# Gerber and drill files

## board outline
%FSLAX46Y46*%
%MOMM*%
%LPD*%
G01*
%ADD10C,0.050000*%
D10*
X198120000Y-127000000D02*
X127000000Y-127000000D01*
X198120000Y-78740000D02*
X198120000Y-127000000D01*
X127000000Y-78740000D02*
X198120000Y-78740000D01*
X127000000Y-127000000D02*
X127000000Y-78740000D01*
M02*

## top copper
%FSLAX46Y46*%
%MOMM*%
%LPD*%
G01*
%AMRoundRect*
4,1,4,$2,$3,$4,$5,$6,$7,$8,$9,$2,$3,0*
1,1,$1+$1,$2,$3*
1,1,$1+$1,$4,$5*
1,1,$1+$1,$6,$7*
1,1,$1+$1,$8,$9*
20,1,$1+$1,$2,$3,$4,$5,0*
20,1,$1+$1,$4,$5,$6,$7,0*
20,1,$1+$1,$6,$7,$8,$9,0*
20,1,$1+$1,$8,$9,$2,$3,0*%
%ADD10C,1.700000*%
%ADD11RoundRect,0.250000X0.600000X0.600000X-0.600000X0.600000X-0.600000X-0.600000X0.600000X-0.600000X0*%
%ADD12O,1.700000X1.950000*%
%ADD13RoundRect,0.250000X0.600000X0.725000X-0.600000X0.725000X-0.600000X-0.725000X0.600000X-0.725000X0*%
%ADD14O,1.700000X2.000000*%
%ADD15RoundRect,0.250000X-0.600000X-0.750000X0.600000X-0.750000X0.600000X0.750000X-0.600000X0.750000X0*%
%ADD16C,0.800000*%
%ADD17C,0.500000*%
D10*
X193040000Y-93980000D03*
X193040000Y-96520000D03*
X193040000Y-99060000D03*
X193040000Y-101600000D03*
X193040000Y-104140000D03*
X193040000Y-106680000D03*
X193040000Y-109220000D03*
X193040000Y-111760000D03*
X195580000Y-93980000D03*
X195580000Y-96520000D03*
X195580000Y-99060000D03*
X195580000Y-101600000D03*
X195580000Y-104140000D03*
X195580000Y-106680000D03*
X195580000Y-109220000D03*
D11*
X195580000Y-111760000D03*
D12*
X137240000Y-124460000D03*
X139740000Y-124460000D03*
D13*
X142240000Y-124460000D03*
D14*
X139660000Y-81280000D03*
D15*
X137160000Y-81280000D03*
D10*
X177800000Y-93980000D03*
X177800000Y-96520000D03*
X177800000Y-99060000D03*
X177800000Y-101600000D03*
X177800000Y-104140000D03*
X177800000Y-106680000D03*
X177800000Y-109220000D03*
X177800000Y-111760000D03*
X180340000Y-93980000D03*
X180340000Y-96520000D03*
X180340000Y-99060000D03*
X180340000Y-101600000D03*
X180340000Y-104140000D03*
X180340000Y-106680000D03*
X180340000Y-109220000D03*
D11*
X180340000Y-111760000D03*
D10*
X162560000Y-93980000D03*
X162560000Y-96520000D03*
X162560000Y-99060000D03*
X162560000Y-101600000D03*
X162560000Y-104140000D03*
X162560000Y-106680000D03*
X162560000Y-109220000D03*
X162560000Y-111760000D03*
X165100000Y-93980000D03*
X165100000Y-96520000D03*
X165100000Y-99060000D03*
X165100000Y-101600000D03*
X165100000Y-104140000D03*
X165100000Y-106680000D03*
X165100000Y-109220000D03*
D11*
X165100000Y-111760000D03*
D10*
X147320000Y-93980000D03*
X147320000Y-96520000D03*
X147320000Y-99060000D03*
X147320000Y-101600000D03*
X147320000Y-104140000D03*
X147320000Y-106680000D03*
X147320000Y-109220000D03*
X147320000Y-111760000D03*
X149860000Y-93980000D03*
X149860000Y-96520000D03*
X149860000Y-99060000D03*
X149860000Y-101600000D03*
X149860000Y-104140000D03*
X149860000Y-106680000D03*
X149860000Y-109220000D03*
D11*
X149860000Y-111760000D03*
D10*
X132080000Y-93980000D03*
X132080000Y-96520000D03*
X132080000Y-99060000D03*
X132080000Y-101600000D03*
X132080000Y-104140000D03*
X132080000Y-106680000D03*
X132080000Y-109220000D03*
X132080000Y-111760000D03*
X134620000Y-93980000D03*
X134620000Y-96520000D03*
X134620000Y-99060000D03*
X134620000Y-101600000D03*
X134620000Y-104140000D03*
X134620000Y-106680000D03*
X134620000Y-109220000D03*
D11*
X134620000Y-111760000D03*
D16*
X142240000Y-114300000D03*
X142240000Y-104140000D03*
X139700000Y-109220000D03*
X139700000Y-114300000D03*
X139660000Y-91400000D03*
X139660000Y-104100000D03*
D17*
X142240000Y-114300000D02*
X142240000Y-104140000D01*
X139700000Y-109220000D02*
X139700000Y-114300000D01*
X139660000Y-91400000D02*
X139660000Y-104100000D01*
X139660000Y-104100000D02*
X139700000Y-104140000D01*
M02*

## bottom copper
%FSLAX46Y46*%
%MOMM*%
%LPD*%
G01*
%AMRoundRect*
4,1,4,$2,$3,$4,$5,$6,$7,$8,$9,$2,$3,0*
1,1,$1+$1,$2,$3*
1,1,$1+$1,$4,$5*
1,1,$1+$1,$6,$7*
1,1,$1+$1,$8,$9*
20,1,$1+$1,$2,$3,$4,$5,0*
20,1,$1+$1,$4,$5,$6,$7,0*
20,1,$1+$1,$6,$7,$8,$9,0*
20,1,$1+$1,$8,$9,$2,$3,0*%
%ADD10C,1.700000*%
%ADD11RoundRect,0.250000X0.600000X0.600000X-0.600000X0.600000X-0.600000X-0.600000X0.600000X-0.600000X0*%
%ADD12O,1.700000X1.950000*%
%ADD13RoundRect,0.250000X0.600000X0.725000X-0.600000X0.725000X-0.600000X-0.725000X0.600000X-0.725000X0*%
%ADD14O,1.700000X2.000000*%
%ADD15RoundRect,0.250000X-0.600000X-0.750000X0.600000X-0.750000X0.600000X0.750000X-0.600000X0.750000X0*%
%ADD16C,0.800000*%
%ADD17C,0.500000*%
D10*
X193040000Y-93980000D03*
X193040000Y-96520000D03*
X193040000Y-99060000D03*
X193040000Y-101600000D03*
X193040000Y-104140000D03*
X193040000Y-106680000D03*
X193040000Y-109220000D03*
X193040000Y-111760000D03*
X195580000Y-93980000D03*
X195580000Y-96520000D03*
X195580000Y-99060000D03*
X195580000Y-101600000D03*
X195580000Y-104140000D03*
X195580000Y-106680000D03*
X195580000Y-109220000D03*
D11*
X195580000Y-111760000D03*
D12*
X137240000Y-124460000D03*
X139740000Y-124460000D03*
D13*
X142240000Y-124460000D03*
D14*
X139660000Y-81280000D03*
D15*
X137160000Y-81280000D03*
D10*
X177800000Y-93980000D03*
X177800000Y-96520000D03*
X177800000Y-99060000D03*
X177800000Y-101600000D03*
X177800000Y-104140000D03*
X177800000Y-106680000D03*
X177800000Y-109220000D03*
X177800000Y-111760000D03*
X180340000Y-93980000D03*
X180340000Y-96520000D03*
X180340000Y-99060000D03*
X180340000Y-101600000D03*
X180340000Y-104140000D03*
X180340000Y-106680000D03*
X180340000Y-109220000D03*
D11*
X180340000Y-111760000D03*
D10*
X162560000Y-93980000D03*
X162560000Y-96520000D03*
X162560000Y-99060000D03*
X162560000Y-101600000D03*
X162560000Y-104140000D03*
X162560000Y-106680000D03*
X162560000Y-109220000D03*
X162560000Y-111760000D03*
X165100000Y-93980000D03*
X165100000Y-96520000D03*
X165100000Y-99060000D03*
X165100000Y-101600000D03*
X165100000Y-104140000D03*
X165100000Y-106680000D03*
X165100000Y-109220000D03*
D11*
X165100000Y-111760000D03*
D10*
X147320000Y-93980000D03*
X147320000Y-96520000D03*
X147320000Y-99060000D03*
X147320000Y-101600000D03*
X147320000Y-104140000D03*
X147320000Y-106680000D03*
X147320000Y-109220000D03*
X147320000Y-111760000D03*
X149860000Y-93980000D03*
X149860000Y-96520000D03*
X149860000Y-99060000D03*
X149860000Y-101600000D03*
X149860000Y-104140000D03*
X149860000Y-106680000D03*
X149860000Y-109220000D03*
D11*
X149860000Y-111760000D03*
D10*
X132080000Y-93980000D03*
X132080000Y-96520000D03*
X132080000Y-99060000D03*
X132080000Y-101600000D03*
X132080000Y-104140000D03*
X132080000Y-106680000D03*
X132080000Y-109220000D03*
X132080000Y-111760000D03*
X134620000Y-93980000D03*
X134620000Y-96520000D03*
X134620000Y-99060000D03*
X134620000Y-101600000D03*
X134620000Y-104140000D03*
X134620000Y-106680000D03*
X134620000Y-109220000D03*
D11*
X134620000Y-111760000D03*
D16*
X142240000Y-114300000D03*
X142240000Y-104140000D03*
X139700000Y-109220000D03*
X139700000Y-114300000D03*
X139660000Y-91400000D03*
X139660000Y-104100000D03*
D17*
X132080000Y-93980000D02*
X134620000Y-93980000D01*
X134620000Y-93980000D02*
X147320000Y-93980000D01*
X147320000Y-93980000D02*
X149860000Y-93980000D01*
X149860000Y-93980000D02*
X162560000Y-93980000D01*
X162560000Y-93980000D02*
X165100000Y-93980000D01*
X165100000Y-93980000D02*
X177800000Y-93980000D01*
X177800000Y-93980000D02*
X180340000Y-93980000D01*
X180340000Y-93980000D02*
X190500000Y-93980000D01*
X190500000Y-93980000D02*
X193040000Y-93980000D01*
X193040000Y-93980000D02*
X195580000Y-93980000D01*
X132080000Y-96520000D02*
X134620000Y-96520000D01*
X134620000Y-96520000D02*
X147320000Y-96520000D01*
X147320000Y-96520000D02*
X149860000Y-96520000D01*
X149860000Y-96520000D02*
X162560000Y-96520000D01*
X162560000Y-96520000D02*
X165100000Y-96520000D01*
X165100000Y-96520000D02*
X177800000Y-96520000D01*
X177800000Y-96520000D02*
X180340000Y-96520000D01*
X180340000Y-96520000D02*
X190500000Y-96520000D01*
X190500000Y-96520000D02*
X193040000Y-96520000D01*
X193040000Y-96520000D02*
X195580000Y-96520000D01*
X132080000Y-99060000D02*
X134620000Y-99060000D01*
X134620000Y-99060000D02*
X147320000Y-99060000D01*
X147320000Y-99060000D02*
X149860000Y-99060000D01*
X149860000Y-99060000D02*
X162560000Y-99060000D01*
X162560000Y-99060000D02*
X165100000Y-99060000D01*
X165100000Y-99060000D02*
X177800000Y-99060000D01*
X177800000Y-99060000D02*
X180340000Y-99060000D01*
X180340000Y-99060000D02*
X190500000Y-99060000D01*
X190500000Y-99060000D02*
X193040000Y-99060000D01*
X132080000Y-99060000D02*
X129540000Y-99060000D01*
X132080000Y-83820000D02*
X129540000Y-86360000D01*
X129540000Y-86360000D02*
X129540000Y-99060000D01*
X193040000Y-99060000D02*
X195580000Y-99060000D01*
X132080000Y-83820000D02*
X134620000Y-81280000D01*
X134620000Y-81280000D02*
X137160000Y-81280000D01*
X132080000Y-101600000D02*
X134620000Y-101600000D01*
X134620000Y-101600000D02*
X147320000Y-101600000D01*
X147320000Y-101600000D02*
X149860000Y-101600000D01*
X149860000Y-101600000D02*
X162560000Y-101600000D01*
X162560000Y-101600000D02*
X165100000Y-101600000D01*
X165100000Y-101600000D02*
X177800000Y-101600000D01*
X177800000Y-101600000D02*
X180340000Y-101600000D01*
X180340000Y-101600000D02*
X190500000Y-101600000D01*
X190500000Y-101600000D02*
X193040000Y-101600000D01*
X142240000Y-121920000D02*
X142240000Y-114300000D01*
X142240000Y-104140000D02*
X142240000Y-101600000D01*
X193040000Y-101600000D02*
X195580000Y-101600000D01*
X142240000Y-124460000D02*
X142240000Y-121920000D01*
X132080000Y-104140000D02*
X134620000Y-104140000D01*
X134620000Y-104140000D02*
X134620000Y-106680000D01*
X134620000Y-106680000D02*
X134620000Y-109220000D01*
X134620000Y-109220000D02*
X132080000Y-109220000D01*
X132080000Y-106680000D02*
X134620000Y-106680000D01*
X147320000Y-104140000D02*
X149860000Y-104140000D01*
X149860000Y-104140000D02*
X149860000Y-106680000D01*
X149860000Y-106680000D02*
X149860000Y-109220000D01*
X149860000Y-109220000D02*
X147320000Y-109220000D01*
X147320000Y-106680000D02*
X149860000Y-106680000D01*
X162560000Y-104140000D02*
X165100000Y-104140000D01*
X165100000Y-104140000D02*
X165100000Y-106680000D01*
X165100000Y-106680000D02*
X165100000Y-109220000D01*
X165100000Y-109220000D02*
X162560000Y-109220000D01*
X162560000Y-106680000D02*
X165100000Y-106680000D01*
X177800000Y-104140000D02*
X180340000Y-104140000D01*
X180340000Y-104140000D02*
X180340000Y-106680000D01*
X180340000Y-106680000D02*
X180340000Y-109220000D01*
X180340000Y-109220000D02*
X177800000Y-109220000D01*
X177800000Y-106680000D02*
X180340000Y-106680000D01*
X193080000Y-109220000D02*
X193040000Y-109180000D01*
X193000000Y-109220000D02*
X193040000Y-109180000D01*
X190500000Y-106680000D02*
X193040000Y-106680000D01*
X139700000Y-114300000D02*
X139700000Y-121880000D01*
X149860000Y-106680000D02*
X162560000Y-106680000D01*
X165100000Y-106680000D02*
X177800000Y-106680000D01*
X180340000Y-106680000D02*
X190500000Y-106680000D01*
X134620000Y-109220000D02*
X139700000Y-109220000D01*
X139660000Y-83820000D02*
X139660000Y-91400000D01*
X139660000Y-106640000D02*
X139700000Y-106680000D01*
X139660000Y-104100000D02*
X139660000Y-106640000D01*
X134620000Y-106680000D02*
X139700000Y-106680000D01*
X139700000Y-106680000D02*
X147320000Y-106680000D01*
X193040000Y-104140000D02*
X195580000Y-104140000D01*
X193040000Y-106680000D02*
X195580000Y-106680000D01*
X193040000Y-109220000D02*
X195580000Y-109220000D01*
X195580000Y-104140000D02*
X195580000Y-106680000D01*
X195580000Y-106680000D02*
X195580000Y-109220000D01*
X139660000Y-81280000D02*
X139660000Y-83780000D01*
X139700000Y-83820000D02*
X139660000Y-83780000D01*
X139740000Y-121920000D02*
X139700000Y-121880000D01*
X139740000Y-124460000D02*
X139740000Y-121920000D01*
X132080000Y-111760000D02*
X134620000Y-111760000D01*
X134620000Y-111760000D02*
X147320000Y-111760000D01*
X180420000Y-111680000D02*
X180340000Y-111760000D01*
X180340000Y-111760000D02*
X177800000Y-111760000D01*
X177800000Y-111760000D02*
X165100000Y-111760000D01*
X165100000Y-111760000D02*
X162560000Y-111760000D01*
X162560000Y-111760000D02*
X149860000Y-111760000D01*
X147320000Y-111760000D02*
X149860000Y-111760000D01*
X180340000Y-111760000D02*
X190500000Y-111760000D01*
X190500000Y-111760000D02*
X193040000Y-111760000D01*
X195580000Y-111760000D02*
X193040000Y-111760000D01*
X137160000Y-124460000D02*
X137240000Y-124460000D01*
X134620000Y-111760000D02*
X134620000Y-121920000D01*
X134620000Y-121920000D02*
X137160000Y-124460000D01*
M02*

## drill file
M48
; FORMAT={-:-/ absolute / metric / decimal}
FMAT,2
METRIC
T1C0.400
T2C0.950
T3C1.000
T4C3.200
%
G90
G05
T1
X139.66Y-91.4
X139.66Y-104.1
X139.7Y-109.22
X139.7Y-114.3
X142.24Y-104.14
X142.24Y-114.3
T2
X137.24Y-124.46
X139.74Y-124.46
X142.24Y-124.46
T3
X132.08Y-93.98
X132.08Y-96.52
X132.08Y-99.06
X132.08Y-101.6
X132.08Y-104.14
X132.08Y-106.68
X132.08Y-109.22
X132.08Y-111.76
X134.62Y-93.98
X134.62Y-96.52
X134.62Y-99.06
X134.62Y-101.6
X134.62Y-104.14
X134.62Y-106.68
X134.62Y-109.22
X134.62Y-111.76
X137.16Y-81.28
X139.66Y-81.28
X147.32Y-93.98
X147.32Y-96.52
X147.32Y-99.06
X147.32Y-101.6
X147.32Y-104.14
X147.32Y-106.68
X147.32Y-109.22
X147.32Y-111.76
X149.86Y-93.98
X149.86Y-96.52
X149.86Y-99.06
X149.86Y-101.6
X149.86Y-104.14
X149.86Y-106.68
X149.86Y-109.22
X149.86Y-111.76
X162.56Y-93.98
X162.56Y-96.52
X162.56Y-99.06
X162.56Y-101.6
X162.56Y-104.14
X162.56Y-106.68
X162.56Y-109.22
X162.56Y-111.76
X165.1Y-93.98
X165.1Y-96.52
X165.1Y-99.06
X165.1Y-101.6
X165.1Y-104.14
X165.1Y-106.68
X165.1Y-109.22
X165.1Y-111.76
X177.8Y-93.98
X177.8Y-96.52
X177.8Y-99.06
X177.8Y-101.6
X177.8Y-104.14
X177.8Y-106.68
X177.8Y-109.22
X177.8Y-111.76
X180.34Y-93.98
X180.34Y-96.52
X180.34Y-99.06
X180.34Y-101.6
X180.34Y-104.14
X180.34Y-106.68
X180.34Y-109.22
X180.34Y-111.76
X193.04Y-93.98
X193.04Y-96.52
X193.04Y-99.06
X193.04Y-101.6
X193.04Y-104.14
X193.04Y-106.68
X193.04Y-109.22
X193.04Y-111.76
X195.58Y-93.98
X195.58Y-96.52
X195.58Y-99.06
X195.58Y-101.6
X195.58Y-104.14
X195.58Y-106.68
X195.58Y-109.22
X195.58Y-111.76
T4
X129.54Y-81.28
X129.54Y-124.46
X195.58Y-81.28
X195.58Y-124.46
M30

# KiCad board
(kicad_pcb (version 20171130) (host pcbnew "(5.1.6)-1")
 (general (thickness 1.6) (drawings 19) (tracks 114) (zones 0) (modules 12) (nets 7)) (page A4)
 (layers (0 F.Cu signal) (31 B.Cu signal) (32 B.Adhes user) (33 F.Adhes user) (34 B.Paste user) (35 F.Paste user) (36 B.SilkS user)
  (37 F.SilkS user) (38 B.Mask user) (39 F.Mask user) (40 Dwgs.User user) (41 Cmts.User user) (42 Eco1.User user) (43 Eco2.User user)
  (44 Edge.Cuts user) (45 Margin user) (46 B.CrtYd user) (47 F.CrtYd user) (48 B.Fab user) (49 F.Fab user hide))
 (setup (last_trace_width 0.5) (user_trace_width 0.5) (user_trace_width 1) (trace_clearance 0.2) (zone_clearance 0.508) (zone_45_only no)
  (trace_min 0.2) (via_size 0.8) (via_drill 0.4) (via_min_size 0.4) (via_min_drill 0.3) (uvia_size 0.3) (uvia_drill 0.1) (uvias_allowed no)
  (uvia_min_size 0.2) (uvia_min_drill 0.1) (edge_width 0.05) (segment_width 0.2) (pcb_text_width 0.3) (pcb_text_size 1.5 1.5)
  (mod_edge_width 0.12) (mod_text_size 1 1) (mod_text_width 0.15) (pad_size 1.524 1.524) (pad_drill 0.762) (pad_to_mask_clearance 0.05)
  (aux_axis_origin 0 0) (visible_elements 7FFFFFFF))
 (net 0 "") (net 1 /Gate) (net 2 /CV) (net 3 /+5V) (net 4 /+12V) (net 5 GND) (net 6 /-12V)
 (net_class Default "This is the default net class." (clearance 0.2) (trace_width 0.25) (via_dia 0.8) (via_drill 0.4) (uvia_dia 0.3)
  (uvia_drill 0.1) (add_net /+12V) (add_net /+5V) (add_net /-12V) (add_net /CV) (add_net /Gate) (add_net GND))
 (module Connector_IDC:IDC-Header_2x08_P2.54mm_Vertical (layer F.Cu) (at 195.58 111.76 180)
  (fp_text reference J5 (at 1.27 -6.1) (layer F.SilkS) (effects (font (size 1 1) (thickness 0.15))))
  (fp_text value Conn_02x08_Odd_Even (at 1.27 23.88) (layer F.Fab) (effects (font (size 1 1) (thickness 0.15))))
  (pad 16 thru_hole circle (at 2.54 17.78 180) (size 1.7 1.7) (drill 1) (layers *.Cu *.Mask) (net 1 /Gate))
  (pad 14 thru_hole circle (at 2.54 15.24 180) (size 1.7 1.7) (drill 1) (layers *.Cu *.Mask) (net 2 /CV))
  (pad 12 thru_hole circle (at 2.54 12.7 180) (size 1.7 1.7) (drill 1) (layers *.Cu *.Mask) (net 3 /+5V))
  (pad 10 thru_hole circle (at 2.54 10.16 180) (size 1.7 1.7) (drill 1) (layers *.Cu *.Mask) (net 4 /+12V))
  (pad 8 thru_hole circle (at 2.54 7.62 180) (size 1.7 1.7) (drill 1) (layers *.Cu *.Mask) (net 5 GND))
  (pad 6 thru_hole circle (at 2.54 5.08 180) (size 1.7 1.7) (drill 1) (layers *.Cu *.Mask) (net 5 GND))
  (pad 4 thru_hole circle (at 2.54 2.54 180) (size 1.7 1.7) (drill 1) (layers *.Cu *.Mask) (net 5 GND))
  (pad 2 thru_hole circle (at 2.54 0 180) (size 1.7 1.7) (drill 1) (layers *.Cu *.Mask) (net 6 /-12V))
  (pad 15 thru_hole circle (at 0 17.78 180) (size 1.7 1.7) (drill 1) (layers *.Cu *.Mask) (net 1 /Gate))
  (pad 13 thru_hole circle (at 0 15.24 180) (size 1.7 1.7) (drill 1) (layers *.Cu *.Mask) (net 2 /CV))
  (pad 11 thru_hole circle (at 0 12.7 180) (size 1.7 1.7) (drill 1) (layers *.Cu *.Mask) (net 3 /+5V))
  (pad 9 thru_hole circle (at 0 10.16 180) (size 1.7 1.7) (drill 1) (layers *.Cu *.Mask) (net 4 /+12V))
  (pad 7 thru_hole circle (at 0 7.62 180) (size 1.7 1.7) (drill 1) (layers *.Cu *.Mask) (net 5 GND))
  (pad 5 thru_hole circle (at 0 5.08 180) (size 1.7 1.7) (drill 1) (layers *.Cu *.Mask) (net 5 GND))
  (pad 3 thru_hole circle (at 0 2.54 180) (size 1.7 1.7) (drill 1) (layers *.Cu *.Mask) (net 5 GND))
  (pad 1 thru_hole roundrect (at 0 0 180) (size 1.7 1.7) (drill 1) (layers *.Cu *.Mask) (roundrect_rratio 0.147059) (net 6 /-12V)))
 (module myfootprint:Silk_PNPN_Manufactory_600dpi (layer F.Cu) (at 182.88 83.82)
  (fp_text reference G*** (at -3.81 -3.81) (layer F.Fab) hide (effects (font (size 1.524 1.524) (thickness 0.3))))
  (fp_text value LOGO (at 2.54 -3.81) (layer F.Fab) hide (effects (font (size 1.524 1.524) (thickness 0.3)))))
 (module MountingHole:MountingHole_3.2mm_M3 (layer F.Cu) (at 195.58 124.46)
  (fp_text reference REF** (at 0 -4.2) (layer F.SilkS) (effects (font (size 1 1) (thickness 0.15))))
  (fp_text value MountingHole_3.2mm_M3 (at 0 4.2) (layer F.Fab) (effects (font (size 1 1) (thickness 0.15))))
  (pad 1 np_thru_hole circle (at 0 0) (size 3.2 3.2) (drill 3.2) (layers *.Cu *.Mask)))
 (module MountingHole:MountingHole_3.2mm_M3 (layer F.Cu) (at 129.54 124.46)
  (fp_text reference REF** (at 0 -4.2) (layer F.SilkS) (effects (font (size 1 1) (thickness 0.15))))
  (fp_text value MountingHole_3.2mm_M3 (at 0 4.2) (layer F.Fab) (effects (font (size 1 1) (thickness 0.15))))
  (pad 1 np_thru_hole circle (at 0 0) (size 3.2 3.2) (drill 3.2) (layers *.Cu *.Mask)))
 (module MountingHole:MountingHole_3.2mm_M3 (layer F.Cu) (at 195.58 81.28)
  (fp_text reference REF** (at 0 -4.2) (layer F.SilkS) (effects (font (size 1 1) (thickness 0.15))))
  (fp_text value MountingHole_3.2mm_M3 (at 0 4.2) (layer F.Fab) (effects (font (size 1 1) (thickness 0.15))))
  (pad 1 np_thru_hole circle (at 0 0) (size 3.2 3.2) (drill 3.2) (layers *.Cu *.Mask)))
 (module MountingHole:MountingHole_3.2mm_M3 (layer F.Cu) (at 129.54 81.28)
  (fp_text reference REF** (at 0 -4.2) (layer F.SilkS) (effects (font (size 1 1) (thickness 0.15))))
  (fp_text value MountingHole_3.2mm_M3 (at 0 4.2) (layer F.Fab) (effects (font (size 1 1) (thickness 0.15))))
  (pad 1 np_thru_hole circle (at 0 0) (size 3.2 3.2) (drill 3.2) (layers *.Cu *.Mask)))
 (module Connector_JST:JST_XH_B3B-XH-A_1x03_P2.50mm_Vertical (layer F.Cu) (at 142.24 124.46 180)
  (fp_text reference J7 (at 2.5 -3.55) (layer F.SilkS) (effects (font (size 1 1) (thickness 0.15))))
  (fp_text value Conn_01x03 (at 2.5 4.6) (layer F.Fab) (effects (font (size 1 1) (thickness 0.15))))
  (pad 3 thru_hole oval (at 5 0 180) (size 1.7 1.95) (drill 0.95) (layers *.Cu *.Mask) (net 6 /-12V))
  (pad 2 thru_hole oval (at 2.5 0 180) (size 1.7 1.95) (drill 0.95) (layers *.Cu *.Mask) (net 5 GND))
  (pad 1 thru_hole roundrect (at 0 0 180) (size 1.7 1.95) (drill 0.95) (layers *.Cu *.Mask) (roundrect_rratio 0.147059) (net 4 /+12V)))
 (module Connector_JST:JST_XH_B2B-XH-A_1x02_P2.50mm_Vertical (layer F.Cu) (at 137.16 81.28)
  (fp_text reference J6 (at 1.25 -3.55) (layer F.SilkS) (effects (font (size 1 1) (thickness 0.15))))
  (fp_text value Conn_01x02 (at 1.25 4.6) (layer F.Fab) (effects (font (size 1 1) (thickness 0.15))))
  (pad 2 thru_hole oval (at 2.5 0) (size 1.7 2) (drill 1) (layers *.Cu *.Mask) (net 5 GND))
  (pad 1 thru_hole roundrect (at 0 0) (size 1.7 2) (drill 1) (layers *.Cu *.Mask) (roundrect_rratio 0.147059) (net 3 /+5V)))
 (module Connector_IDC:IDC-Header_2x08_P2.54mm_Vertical (layer F.Cu) (at 180.34 111.76 180)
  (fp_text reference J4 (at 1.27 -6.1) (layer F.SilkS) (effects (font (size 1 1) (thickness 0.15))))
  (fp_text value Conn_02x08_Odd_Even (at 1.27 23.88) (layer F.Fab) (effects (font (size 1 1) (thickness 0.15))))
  (pad 16 thru_hole circle (at 2.54 17.78 180) (size 1.7 1.7) (drill 1) (layers *.Cu *.Mask) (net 1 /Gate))
  (pad 14 thru_hole circle (at 2.54 15.24 180) (size 1.7 1.7) (drill 1) (layers *.Cu *.Mask) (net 2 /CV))
  (pad 12 thru_hole circle (at 2.54 12.7 180) (size 1.7 1.7) (drill 1) (layers *.Cu *.Mask) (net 3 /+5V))
  (pad 10 thru_hole circle (at 2.54 10.16 180) (size 1.7 1.7) (drill 1) (layers *.Cu *.Mask) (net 4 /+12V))
  (pad 8 thru_hole circle (at 2.54 7.62 180) (size 1.7 1.7) (drill 1) (layers *.Cu *.Mask) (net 5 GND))
  (pad 6 thru_hole circle (at 2.54 5.08 180) (size 1.7 1.7) (drill 1) (layers *.Cu *.Mask) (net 5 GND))
  (pad 4 thru_hole circle (at 2.54 2.54 180) (size 1.7 1.7) (drill 1) (layers *.Cu *.Mask) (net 5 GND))
  (pad 2 thru_hole circle (at 2.54 0 180) (size 1.7 1.7) (drill 1) (layers *.Cu *.Mask) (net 6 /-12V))
  (pad 15 thru_hole circle (at 0 17.78 180) (size 1.7 1.7) (drill 1) (layers *.Cu *.Mask) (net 1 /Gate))
  (pad 13 thru_hole circle (at 0 15.24 180) (size 1.7 1.7) (drill 1) (layers *.Cu *.Mask) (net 2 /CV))
  (pad 11 thru_hole circle (at 0 12.7 180) (size 1.7 1.7) (drill 1) (layers *.Cu *.Mask) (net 3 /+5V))
  (pad 9 thru_hole circle (at 0 10.16 180) (size 1.7 1.7) (drill 1) (layers *.Cu *.Mask) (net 4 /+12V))
  (pad 7 thru_hole circle (at 0 7.62 180) (size 1.7 1.7) (drill 1) (layers *.Cu *.Mask) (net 5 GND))
  (pad 5 thru_hole circle (at 0 5.08 180) (size 1.7 1.7) (drill 1) (layers *.Cu *.Mask) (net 5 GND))
  (pad 3 thru_hole circle (at 0 2.54 180) (size 1.7 1.7) (drill 1) (layers *.Cu *.Mask) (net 5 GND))
  (pad 1 thru_hole roundrect (at 0 0 180) (size 1.7 1.7) (drill 1) (layers *.Cu *.Mask) (roundrect_rratio 0.147059) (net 6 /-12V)))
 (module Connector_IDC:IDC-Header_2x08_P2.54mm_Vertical (layer F.Cu) (at 165.1 111.76 180)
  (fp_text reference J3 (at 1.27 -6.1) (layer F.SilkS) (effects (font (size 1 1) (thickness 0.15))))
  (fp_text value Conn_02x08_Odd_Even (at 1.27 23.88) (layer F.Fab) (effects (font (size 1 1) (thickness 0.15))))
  (pad 16 thru_hole circle (at 2.54 17.78 180) (size 1.7 1.7) (drill 1) (layers *.Cu *.Mask) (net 1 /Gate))
  (pad 14 thru_hole circle (at 2.54 15.24 180) (size 1.7 1.7) (drill 1) (layers *.Cu *.Mask) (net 2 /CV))
  (pad 12 thru_hole circle (at 2.54 12.7 180) (size 1.7 1.7) (drill 1) (layers *.Cu *.Mask) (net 3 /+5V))
  (pad 10 thru_hole circle (at 2.54 10.16 180) (size 1.7 1.7) (drill 1) (layers *.Cu *.Mask) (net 4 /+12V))
  (pad 8 thru_hole circle (at 2.54 7.62 180) (size 1.7 1.7) (drill 1) (layers *.Cu *.Mask) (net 5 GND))
  (pad 6 thru_hole circle (at 2.54 5.08 180) (size 1.7 1.7) (drill 1) (layers *.Cu *.Mask) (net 5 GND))
  (pad 4 thru_hole circle (at 2.54 2.54 180) (size 1.7 1.7) (drill 1) (layers *.Cu *.Mask) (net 5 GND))
  (pad 2 thru_hole circle (at 2.54 0 180) (size 1.7 1.7) (drill 1) (layers *.Cu *.Mask) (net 6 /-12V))
  (pad 15 thru_hole circle (at 0 17.78 180) (size 1.7 1.7) (drill 1) (layers *.Cu *.Mask) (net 1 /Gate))
  (pad 13 thru_hole circle (at 0 15.24 180) (size 1.7 1.7) (drill 1) (layers *.Cu *.Mask) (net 2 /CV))
  (pad 11 thru_hole circle (at 0 12.7 180) (size 1.7 1.7) (drill 1) (layers *.Cu *.Mask) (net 3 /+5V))
  (pad 9 thru_hole circle (at 0 10.16 180) (size 1.7 1.7) (drill 1) (layers *.Cu *.Mask) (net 4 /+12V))
  (pad 7 thru_hole circle (at 0 7.62 180) (size 1.7 1.7) (drill 1) (layers *.Cu *.Mask) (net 5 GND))
  (pad 5 thru_hole circle (at 0 5.08 180) (size 1.7 1.7) (drill 1) (layers *.Cu *.Mask) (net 5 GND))
  (pad 3 thru_hole circle (at 0 2.54 180) (size 1.7 1.7) (drill 1) (layers *.Cu *.Mask) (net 5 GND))
  (pad 1 thru_hole roundrect (at 0 0 180) (size 1.7 1.7) (drill 1) (layers *.Cu *.Mask) (roundrect_rratio 0.147059) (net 6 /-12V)))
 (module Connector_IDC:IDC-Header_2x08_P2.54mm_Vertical (layer F.Cu) (at 149.86 111.76 180)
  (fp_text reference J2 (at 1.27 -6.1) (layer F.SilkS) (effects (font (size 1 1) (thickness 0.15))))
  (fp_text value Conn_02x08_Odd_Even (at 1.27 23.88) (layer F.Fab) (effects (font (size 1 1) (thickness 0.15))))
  (pad 16 thru_hole circle (at 2.54 17.78 180) (size 1.7 1.7) (drill 1) (layers *.Cu *.Mask) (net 1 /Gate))
  (pad 14 thru_hole circle (at 2.54 15.24 180) (size 1.7 1.7) (drill 1) (layers *.Cu *.Mask) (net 2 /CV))
  (pad 12 thru_hole circle (at 2.54 12.7 180) (size 1.7 1.7) (drill 1) (layers *.Cu *.Mask) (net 3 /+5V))
  (pad 10 thru_hole circle (at 2.54 10.16 180) (size 1.7 1.7) (drill 1) (layers *.Cu *.Mask) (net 4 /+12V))
  (pad 8 thru_hole circle (at 2.54 7.62 180) (size 1.7 1.7) (drill 1) (layers *.Cu *.Mask) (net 5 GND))
  (pad 6 thru_hole circle (at 2.54 5.08 180) (size 1.7 1.7) (drill 1) (layers *.Cu *.Mask) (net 5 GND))
  (pad 4 thru_hole circle (at 2.54 2.54 180) (size 1.7 1.7) (drill 1) (layers *.Cu *.Mask) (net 5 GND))
  (pad 2 thru_hole circle (at 2.54 0 180) (size 1.7 1.7) (drill 1) (layers *.Cu *.Mask) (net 6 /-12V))
  (pad 15 thru_hole circle (at 0 17.78 180) (size 1.7 1.7) (drill 1) (layers *.Cu *.Mask) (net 1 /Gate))
  (pad 13 thru_hole circle (at 0 15.24 180) (size 1.7 1.7) (drill 1) (layers *.Cu *.Mask) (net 2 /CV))
  (pad 11 thru_hole circle (at 0 12.7 180) (size 1.7 1.7) (drill 1) (layers *.Cu *.Mask) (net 3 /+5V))
  (pad 9 thru_hole circle (at 0 10.16 180) (size 1.7 1.7) (drill 1) (layers *.Cu *.Mask) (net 4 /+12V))
  (pad 7 thru_hole circle (at 0 7.62 180) (size 1.7 1.7) (drill 1) (layers *.Cu *.Mask) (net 5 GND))
  (pad 5 thru_hole circle (at 0 5.08 180) (size 1.7 1.7) (drill 1) (layers *.Cu *.Mask) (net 5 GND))
  (pad 3 thru_hole circle (at 0 2.54 180) (size 1.7 1.7) (drill 1) (layers *.Cu *.Mask) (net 5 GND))
  (pad 1 thru_hole roundrect (at 0 0 180) (size 1.7 1.7) (drill 1) (layers *.Cu *.Mask) (roundrect_rratio 0.147059) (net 6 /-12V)))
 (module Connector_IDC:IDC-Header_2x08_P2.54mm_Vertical (layer F.Cu) (at 134.62 111.76 180)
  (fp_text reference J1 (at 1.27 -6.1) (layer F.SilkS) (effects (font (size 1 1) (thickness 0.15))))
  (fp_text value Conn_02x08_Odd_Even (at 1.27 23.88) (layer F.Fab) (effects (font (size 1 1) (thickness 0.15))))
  (pad 16 thru_hole circle (at 2.54 17.78 180) (size 1.7 1.7) (drill 1) (layers *.Cu *.Mask) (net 1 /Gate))
  (pad 14 thru_hole circle (at 2.54 15.24 180) (size 1.7 1.7) (drill 1) (layers *.Cu *.Mask) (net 2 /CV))
  (pad 12 thru_hole circle (at 2.54 12.7 180) (size 1.7 1.7) (drill 1) (layers *.Cu *.Mask) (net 3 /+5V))
  (pad 10 thru_hole circle (at 2.54 10.16 180) (size 1.7 1.7) (drill 1) (layers *.Cu *.Mask) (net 4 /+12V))
  (pad 8 thru_hole circle (at 2.54 7.62 180) (size 1.7 1.7) (drill 1) (layers *.Cu *.Mask) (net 5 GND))
  (pad 6 thru_hole circle (at 2.54 5.08 180) (size 1.7 1.7) (drill 1) (layers *.Cu *.Mask) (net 5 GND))
  (pad 4 thru_hole circle (at 2.54 2.54 180) (size 1.7 1.7) (drill 1) (layers *.Cu *.Mask) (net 5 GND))
  (pad 2 thru_hole circle (at 2.54 0 180) (size 1.7 1.7) (drill 1) (layers *.Cu *.Mask) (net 6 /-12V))
  (pad 15 thru_hole circle (at 0 17.78 180) (size 1.7 1.7) (drill 1) (layers *.Cu *.Mask) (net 1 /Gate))
  (pad 13 thru_hole circle (at 0 15.24 180) (size 1.7 1.7) (drill 1) (layers *.Cu *.Mask) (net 2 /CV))
  (pad 11 thru_hole circle (at 0 12.7 180) (size 1.7 1.7) (drill 1) (layers *.Cu *.Mask) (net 3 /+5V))
  (pad 9 thru_hole circle (at 0 10.16 180) (size 1.7 1.7) (drill 1) (layers *.Cu *.Mask) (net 4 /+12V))
  (pad 7 thru_hole circle (at 0 7.62 180) (size 1.7 1.7) (drill 1) (layers *.Cu *.Mask) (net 5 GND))
  (pad 5 thru_hole circle (at 0 5.08 180) (size 1.7 1.7) (drill 1) (layers *.Cu *.Mask) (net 5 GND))
  (pad 3 thru_hole circle (at 0 2.54 180) (size 1.7 1.7) (drill 1) (layers *.Cu *.Mask) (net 5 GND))
  (pad 1 thru_hole roundrect (at 0 0 180) (size 1.7 1.7) (drill 1) (layers *.Cu *.Mask) (roundrect_rratio 0.147059) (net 6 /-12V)))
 (gr_line (start 198.12 127) (end 127 127) (layer Edge.Cuts) (width 0.05))
 (gr_line (start 198.12 78.74) (end 198.12 127) (layer Edge.Cuts) (width 0.05))
 (gr_line (start 127 78.74) (end 198.12 78.74) (layer Edge.Cuts) (width 0.05))
 (gr_line (start 127 127) (end 127 78.74) (layer Edge.Cuts) (width 0.05))
 (segment (start 132.08 93.98) (end 134.62 93.98) (width 0.5) (layer B.Cu) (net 1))
 (segment (start 134.62 93.98) (end 147.32 93.98) (width 0.5) (layer B.Cu) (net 1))
 (segment (start 147.32 93.98) (end 149.86 93.98) (width 0.5) (layer B.Cu) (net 1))
 (segment (start 149.86 93.98) (end 162.56 93.98) (width 0.5) (layer B.Cu) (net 1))
 (segment (start 162.56 93.98) (end 165.1 93.98) (width 0.5) (layer B.Cu) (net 1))
 (segment (start 165.1 93.98) (end 177.8 93.98) (width 0.5) (layer B.Cu) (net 1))
 (segment (start 177.8 93.98) (end 180.34 93.98) (width 0.5) (layer B.Cu) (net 1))
 (segment (start 180.34 93.98) (end 190.5 93.98) (width 0.5) (layer B.Cu) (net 1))
 (segment (start 190.5 93.98) (end 193.04 93.98) (width 0.5) (layer B.Cu) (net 1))
 (segment (start 193.04 93.98) (end 195.58 93.98) (width 0.5) (layer B.Cu) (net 1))
 (segment (start 132.08 96.52) (end 134.62 96.52) (width 0.5) (layer B.Cu) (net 2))
 (segment (start 134.62 96.52) (end 147.32 96.52) (width 0.5) (layer B.Cu) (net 2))
 (segment (start 147.32 96.52) (end 149.86 96.52) (width 0.5) (layer B.Cu) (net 2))
 (segment (start 149.86 96.52) (end 162.56 96.52) (width 0.5) (layer B.Cu) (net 2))
 (segment (start 162.56 96.52) (end 165.1 96.52) (width 0.5) (layer B.Cu) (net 2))
 (segment (start 165.1 96.52) (end 177.8 96.52) (width 0.5) (layer B.Cu) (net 2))
 (segment (start 177.8 96.52) (end 180.34 96.52) (width 0.5) (layer B.Cu) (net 2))
 (segment (start 180.34 96.52) (end 190.5 96.52) (width 0.5) (layer B.Cu) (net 2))
 (segment (start 190.5 96.52) (end 193.04 96.52) (width 0.5) (layer B.Cu) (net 2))
 (segment (start 193.04 96.52) (end 195.58 96.52) (width 0.5) (layer B.Cu) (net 2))
 (segment (start 132.08 99.06) (end 134.62 99.06) (width 0.5) (layer B.Cu) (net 3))
 (segment (start 134.62 99.06) (end 147.32 99.06) (width 0.5) (layer B.Cu) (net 3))
 (segment (start 147.32 99.06) (end 149.86 99.06) (width 0.5) (layer B.Cu) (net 3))
 (segment (start 149.86 99.06) (end 162.56 99.06) (width 0.5) (layer B.Cu) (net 3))
 (segment (start 162.56 99.06) (end 165.1 99.06) (width 0.5) (layer B.Cu) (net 3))
 (segment (start 165.1 99.06) (end 177.8 99.06) (width 0.5) (layer B.Cu) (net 3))
 (segment (start 177.8 99.06) (end 180.34 99.06) (width 0.5) (layer B.Cu) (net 3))
 (segment (start 180.34 99.06) (end 190.5 99.06) (width 0.5) (layer B.Cu) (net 3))
 (segment (start 190.5 99.06) (end 193.04 99.06) (width 0.5) (layer B.Cu) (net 3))
 (segment (start 132.08 99.06) (end 129.54 99.06) (width 0.5) (layer B.Cu) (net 3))
 (segment (start 132.08 83.82) (end 129.54 86.36) (width 0.5) (layer B.Cu) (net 3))
 (segment (start 129.54 86.36) (end 129.54 99.06) (width 0.5) (layer B.Cu) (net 3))
 (segment (start 193.04 99.06) (end 195.58 99.06) (width 0.5) (layer B.Cu) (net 3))
 (segment (start 132.08 83.82) (end 134.62 81.28) (width 0.5) (layer B.Cu) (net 3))
 (segment (start 134.62 81.28) (end 137.16 81.28) (width 0.5) (layer B.Cu) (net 3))
 (segment (start 132.08 101.6) (end 134.62 101.6) (width 0.5) (layer B.Cu) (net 4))
 (segment (start 134.62 101.6) (end 147.32 101.6) (width 0.5) (layer B.Cu) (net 4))
 (segment (start 147.32 101.6) (end 149.86 101.6) (width 0.5) (layer B.Cu) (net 4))
 (segment (start 149.86 101.6) (end 162.56 101.6) (width 0.5) (layer B.Cu) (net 4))
 (segment (start 162.56 101.6) (end 165.1 101.6) (width 0.5) (layer B.Cu) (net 4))
 (segment (start 165.1 101.6) (end 177.8 101.6) (width 0.5) (layer B.Cu) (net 4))
 (segment (start 177.8 101.6) (end 180.34 101.6) (width 0.5) (layer B.Cu) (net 4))
 (segment (start 180.34 101.6) (end 190.5 101.6) (width 0.5) (layer B.Cu) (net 4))
 (segment (start 190.5 101.6) (end 193.04 101.6) (width 0.5) (layer B.Cu) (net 4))
 (segment (start 142.24 121.92) (end 142.24 114.3) (width 0.5) (layer B.Cu) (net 4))
 (via (at 142.24 114.3) (size 0.8) (drill 0.4) (layers F.Cu B.Cu) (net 4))
 (segment (start 142.24 114.3) (end 142.24 104.14) (width 0.5) (layer F.Cu) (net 4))
 (via (at 142.24 104.14) (size 0.8) (drill 0.4) (layers F.Cu B.Cu) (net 4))
 (segment (start 142.24 104.14) (end 142.24 101.6) (width 0.5) (layer B.Cu) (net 4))
 (segment (start 193.04 101.6) (end 195.58 101.6) (width 0.5) (layer B.Cu) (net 4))
 (segment (start 142.24 124.46) (end 142.24 121.92) (width 0.5) (layer B.Cu) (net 4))
 (segment (start 132.08 104.14) (end 134.62 104.14) (width 0.5) (layer B.Cu) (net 5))
 (segment (start 134.62 104.14) (end 134.62 106.68) (width 0.5) (layer B.Cu) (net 5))
 (segment (start 134.62 106.68) (end 134.62 109.22) (width 0.5) (layer B.Cu) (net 5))
 (segment (start 134.62 109.22) (end 132.08 109.22) (width 0.5) (layer B.Cu) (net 5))
 (segment (start 132.08 106.68) (end 134.62 106.68) (width 0.5) (layer B.Cu) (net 5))
 (segment (start 147.32 104.14) (end 149.86 104.14) (width 0.5) (layer B.Cu) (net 5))
 (segment (start 149.86 104.14) (end 149.86 106.68) (width 0.5) (layer B.Cu) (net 5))
 (segment (start 149.86 106.68) (end 149.86 109.22) (width 0.5) (layer B.Cu) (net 5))
 (segment (start 149.86 109.22) (end 147.32 109.22) (width 0.5) (layer B.Cu) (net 5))
 (segment (start 147.32 106.68) (end 149.86 106.68) (width 0.5) (layer B.Cu) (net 5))
 (segment (start 162.56 104.14) (end 165.1 104.14) (width 0.5) (layer B.Cu) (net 5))
 (segment (start 165.1 104.14) (end 165.1 106.68) (width 0.5) (layer B.Cu) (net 5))
 (segment (start 165.1 106.68) (end 165.1 109.22) (width 0.5) (layer B.Cu) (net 5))
 (segment (start 165.1 109.22) (end 162.56 109.22) (width 0.5) (layer B.Cu) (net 5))
 (segment (start 162.56 106.68) (end 165.1 106.68) (width 0.5) (layer B.Cu) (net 5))
 (segment (start 177.8 104.14) (end 180.34 104.14) (width 0.5) (layer B.Cu) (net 5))
 (segment (start 180.34 104.14) (end 180.34 106.68) (width 0.5) (layer B.Cu) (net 5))
 (segment (start 180.34 106.68) (end 180.34 109.22) (width 0.5) (layer B.Cu) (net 5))
 (segment (start 180.34 109.22) (end 177.8 109.22) (width 0.5) (layer B.Cu) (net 5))
 (segment (start 177.8 106.68) (end 180.34 106.68) (width 0.5) (layer B.Cu) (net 5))
 (segment (start 193.08 109.22) (end 193.04 109.18) (width 0.5) (layer B.Cu) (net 5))
 (segment (start 193 109.22) (end 193.04 109.18) (width 0.5) (layer B.Cu) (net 5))
 (segment (start 190.5 106.68) (end 193.04 106.68) (width 0.5) (layer B.Cu) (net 5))
 (via (at 139.7 109.22) (size 0.8) (drill 0.4) (layers F.Cu B.Cu) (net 5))
 (segment (start 139.7 109.22) (end 139.7 114.3) (width 0.5) (layer F.Cu) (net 5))
 (via (at 139.7 114.3) (size 0.8) (drill 0.4) (layers F.Cu B.Cu) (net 5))
 (segment (start 139.7 114.3) (end 139.7 121.88) (width 0.5) (layer B.Cu) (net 5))
 (segment (start 149.86 106.68) (end 162.56 106.68) (width 0.5) (layer B.Cu) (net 5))
 (segment (start 165.1 106.68) (end 177.8 106.68) (width 0.5) (layer B.Cu) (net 5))
 (segment (start 180.34 106.68) (end 190.5 106.68) (width 0.5) (layer B.Cu) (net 5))
 (segment (start 134.62 109.22) (end 139.7 109.22) (width 0.5) (layer B.Cu) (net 5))
 (segment (start 139.66 83.82) (end 139.66 91.4) (width 0.5) (layer B.Cu) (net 5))
 (via (at 139.66 91.4) (size 0.8) (drill 0.4) (layers F.Cu B.Cu) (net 5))
 (segment (start 139.66 91.4) (end 139.66 104.1) (width 0.5) (layer F.Cu) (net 5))
 (via (at 139.66 104.1) (size 0.8) (drill 0.4) (layers F.Cu B.Cu) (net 5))
 (segment (start 139.66 104.1) (end 139.7 104.14) (width 0.5) (layer F.Cu) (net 5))
 (segment (start 139.66 106.64) (end 139.7 106.68) (width 0.5) (layer B.Cu) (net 5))
 (segment (start 139.66 104.1) (end 139.66 106.64) (width 0.5) (layer B.Cu) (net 5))
 (segment (start 134.62 106.68) (end 139.7 106.68) (width 0.5) (layer B.Cu) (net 5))
 (segment (start 139.7 106.68) (end 147.32 106.68) (width 0.5) (layer B.Cu) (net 5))
 (segment (start 193.04 104.14) (end 195.58 104.14) (width 0.5) (layer B.Cu) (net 5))
 (segment (start 193.04 106.68) (end 195.58 106.68) (width 0.5) (layer B.Cu) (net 5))
 (segment (start 193.04 109.22) (end 195.58 109.22) (width 0.5) (layer B.Cu) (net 5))
 (segment (start 195.58 104.14) (end 195.58 106.68) (width 0.5) (layer B.Cu) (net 5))
 (segment (start 195.58 106.68) (end 195.58 109.22) (width 0.5) (layer B.Cu) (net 5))
 (segment (start 139.66 81.28) (end 139.66 83.78) (width 0.5) (layer B.Cu) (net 5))
 (segment (start 139.7 83.82) (end 139.66 83.78) (width 0.5) (layer B.Cu) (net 5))
 (segment (start 139.74 121.92) (end 139.7 121.88) (width 0.5) (layer B.Cu) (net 5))
 (segment (start 139.74 124.46) (end 139.74 121.92) (width 0.5) (layer B.Cu) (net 5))
 (segment (start 132.08 111.76) (end 134.62 111.76) (width 0.5) (layer B.Cu) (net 6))
 (segment (start 134.62 111.76) (end 147.32 111.76) (width 0.5) (layer B.Cu) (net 6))
 (segment (start 180.42 111.68) (end 180.34 111.76) (width 0.5) (layer B.Cu) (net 6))
 (segment (start 180.34 111.76) (end 177.8 111.76) (width 0.5) (layer B.Cu) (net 6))
 (segment (start 177.8 111.76) (end 165.1 111.76) (width 0.5) (layer B.Cu) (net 6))
 (segment (start 165.1 111.76) (end 162.56 111.76) (width 0.5) (layer B.Cu) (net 6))
 (segment (start 162.56 111.76) (end 149.86 111.76) (width 0.5) (layer B.Cu) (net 6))
 (segment (start 147.32 111.76) (end 149.86 111.76) (width 0.5) (layer B.Cu) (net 6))
 (segment (start 180.34 111.76) (end 190.5 111.76) (width 0.5) (layer B.Cu) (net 6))
 (segment (start 190.5 111.76) (end 193.04 111.76) (width 0.5) (layer B.Cu) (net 6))
 (segment (start 195.58 111.76) (end 193.04 111.76) (width 0.5) (layer B.Cu) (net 6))
 (segment (start 137.16 124.46) (end 137.24 124.46) (width 0.5) (layer B.Cu) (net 6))
 (segment (start 134.62 111.76) (end 134.62 121.92) (width 0.5) (layer B.Cu) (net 6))
 (segment (start 134.62 121.92) (end 137.16 124.46) (width 0.5) (layer B.Cu) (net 6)))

